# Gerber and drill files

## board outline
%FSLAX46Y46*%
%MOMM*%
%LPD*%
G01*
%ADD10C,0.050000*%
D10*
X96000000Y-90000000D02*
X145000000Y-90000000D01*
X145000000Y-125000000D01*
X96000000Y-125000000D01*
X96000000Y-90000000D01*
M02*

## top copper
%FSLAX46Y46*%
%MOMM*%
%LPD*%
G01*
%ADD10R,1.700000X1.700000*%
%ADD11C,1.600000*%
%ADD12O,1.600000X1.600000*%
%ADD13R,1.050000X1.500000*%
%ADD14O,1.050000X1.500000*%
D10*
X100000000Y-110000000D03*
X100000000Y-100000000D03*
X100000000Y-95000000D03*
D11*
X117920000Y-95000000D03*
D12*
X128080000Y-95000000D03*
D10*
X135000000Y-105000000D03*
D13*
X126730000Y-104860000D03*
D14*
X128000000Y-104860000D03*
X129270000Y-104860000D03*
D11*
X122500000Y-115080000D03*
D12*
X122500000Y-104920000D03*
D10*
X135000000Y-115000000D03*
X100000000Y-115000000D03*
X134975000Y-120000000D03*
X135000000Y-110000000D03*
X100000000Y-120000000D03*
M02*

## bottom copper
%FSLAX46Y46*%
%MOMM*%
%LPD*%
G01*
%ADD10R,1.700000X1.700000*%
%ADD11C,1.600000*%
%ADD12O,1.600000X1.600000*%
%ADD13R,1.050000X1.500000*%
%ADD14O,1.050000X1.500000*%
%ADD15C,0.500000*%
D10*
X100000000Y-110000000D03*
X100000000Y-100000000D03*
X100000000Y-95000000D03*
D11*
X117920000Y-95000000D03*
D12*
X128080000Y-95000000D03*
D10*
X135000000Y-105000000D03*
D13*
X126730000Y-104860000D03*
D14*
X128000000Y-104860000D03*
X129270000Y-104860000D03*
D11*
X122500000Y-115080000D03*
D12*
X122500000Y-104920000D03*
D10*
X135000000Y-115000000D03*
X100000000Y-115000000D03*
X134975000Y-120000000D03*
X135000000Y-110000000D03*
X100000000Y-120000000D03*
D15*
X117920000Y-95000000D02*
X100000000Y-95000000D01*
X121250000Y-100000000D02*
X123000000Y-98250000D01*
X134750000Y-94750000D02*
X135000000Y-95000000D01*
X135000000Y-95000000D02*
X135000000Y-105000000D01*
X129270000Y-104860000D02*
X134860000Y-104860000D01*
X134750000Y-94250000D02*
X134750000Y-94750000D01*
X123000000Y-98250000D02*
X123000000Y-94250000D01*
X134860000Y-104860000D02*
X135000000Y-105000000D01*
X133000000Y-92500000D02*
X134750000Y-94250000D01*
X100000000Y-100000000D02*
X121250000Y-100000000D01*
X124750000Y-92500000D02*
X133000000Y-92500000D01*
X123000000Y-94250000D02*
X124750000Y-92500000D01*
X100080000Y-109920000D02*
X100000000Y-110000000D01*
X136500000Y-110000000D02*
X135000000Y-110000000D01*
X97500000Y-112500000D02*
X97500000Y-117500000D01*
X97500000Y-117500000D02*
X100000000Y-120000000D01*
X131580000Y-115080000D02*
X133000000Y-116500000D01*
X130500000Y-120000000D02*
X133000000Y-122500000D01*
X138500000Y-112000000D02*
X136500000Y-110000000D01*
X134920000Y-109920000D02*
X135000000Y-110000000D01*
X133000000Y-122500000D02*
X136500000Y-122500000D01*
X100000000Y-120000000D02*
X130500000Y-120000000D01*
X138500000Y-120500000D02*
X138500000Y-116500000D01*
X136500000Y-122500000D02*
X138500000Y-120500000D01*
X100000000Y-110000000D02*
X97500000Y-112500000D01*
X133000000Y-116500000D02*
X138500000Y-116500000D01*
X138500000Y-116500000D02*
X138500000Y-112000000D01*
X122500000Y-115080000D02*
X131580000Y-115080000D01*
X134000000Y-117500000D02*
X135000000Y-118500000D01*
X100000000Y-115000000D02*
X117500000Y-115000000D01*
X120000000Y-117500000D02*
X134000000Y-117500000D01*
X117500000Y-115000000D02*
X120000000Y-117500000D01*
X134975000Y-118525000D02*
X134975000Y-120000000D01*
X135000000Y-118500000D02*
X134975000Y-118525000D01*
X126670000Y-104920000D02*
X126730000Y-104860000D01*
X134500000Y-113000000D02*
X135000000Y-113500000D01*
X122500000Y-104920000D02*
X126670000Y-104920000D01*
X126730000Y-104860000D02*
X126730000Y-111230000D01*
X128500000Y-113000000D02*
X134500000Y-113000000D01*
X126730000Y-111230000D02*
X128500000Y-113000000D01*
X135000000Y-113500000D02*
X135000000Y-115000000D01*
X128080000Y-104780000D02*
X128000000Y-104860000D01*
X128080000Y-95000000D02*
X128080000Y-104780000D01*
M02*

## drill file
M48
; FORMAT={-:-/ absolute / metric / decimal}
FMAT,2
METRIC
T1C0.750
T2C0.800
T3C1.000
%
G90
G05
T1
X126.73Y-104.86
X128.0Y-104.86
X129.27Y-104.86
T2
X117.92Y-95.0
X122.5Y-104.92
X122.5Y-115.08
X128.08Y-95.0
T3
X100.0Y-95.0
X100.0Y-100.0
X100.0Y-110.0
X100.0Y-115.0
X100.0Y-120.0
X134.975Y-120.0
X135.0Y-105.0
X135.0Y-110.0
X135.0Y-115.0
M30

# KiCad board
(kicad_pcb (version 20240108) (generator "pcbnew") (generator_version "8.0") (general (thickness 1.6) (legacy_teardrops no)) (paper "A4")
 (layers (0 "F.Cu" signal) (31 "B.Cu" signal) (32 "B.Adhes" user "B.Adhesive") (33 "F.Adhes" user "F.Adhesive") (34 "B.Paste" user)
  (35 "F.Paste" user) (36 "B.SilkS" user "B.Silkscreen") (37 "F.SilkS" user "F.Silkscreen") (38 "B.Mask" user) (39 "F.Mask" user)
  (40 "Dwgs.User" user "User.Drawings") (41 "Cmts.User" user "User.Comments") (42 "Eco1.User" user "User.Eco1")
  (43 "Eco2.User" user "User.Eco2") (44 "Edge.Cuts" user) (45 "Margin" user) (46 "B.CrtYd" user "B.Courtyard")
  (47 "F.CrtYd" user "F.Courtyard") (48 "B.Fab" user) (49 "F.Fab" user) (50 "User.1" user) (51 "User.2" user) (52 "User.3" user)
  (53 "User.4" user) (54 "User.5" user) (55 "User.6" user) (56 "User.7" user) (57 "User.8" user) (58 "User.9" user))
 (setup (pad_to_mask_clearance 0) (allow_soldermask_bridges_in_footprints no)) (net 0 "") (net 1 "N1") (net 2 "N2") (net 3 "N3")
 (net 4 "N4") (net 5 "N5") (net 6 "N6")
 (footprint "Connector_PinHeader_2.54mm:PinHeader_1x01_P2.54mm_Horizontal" (layer "F.Cu") (at 100 110 180)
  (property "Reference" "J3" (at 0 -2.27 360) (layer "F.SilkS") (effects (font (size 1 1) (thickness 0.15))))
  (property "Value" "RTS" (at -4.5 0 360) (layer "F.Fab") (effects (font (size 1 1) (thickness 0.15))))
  (pad "1" thru_hole rect (at 0 0 180) (size 1.7 1.7) (drill 1) (layers "*.Cu" "*.Mask") (remove_unused_layers no) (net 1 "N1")))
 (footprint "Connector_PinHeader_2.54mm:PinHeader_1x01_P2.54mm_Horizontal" (layer "F.Cu") (at 100 100 180)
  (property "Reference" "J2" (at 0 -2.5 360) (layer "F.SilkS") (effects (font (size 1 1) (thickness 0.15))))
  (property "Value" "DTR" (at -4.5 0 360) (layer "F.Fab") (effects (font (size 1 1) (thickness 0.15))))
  (pad "1" thru_hole rect (at 0 0 180) (size 1.7 1.7) (drill 1) (layers "*.Cu" "*.Mask") (remove_unused_layers no) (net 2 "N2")))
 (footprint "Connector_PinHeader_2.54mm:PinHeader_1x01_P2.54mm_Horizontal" (layer "F.Cu") (at 100 95 180)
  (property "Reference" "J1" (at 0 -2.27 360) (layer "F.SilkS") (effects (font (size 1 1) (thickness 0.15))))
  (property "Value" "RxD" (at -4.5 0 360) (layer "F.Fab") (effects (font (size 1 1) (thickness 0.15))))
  (pad "1" thru_hole rect (at 0 0 180) (size 1.7 1.7) (drill 1) (layers "*.Cu" "*.Mask") (remove_unused_layers no) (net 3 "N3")))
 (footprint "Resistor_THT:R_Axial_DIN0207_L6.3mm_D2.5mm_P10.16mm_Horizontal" (layer "F.Cu") (at 117.92 95)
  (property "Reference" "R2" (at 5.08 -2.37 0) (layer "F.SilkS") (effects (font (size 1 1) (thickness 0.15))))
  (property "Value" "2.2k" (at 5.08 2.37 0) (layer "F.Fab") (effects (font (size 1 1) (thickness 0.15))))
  (pad "1" thru_hole circle (at 0 0) (size 1.6 1.6) (drill 0.8) (layers "*.Cu" "*.Mask") (remove_unused_layers no) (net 3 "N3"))
  (pad "2" thru_hole oval (at 10.16 0) (size 1.6 1.6) (drill 0.8) (layers "*.Cu" "*.Mask") (remove_unused_layers no) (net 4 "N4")))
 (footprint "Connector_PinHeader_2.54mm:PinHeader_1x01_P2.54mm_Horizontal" (layer "F.Cu") (at 135 105)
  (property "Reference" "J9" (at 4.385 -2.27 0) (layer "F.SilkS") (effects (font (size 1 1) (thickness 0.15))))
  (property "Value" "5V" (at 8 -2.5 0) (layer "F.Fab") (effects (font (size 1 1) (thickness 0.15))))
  (pad "1" thru_hole rect (at 0 0) (size 1.7 1.7) (drill 1) (layers "*.Cu" "*.Mask") (remove_unused_layers no) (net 2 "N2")))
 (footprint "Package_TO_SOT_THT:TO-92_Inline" (layer "F.Cu") (at 126.73 104.86)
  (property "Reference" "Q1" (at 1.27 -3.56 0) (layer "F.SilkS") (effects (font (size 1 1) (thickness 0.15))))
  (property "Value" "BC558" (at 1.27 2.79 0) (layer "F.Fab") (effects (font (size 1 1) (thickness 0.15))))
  (pad "1" thru_hole rect (at 0 0) (size 1.05 1.5) (drill 0.75) (layers "*.Cu" "*.Mask") (remove_unused_layers no) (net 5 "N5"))
  (pad "2" thru_hole oval (at 1.27 0) (size 1.05 1.5) (drill 0.75) (layers "*.Cu" "*.Mask") (remove_unused_layers no) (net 4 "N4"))
  (pad "3" thru_hole oval (at 2.54 0) (size 1.05 1.5) (drill 0.75) (layers "*.Cu" "*.Mask") (remove_unused_layers no) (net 2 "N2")))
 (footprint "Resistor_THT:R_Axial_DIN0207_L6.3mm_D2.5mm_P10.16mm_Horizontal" (layer "F.Cu") (at 122.5 115.08 90)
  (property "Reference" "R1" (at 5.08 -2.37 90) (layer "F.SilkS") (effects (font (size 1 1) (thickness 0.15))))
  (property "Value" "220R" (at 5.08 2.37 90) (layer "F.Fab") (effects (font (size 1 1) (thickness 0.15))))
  (pad "1" thru_hole circle (at 0 0 90) (size 1.6 1.6) (drill 0.8) (layers "*.Cu" "*.Mask") (remove_unused_layers no) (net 1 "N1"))
  (pad "2" thru_hole oval (at 10.16 0 90) (size 1.6 1.6) (drill 0.8) (layers "*.Cu" "*.Mask") (remove_unused_layers no) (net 5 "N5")))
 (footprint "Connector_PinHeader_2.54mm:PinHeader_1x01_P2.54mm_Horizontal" (layer "F.Cu") (at 135 115)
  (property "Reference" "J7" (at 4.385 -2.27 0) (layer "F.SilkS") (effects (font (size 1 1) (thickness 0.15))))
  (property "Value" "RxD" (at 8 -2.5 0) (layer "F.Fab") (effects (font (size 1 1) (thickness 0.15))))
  (pad "1" thru_hole rect (at 0 0) (size 1.7 1.7) (drill 1) (layers "*.Cu" "*.Mask") (remove_unused_layers no) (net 5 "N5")))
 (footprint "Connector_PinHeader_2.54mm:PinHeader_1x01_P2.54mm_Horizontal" (layer "F.Cu") (at 100 115 180)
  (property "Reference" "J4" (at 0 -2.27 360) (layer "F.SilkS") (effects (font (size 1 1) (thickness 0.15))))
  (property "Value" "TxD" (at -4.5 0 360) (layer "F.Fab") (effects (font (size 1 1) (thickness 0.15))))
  (pad "1" thru_hole rect (at 0 0 180) (size 1.7 1.7) (drill 1) (layers "*.Cu" "*.Mask") (remove_unused_layers no) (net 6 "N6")))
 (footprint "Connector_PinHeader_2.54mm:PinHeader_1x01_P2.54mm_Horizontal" (layer "F.Cu") (at 134.975 120)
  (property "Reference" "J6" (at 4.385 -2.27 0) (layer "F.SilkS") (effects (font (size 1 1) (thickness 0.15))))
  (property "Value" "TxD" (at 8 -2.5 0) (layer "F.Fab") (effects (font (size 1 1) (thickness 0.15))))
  (pad "1" thru_hole rect (at 0 0) (size 1.7 1.7) (drill 1) (layers "*.Cu" "*.Mask") (remove_unused_layers no) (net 6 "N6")))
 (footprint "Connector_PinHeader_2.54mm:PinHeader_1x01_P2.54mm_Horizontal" (layer "F.Cu") (at 135 110)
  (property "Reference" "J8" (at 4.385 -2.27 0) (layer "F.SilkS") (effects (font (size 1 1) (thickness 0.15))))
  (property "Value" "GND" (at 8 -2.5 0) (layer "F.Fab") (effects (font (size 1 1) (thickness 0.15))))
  (pad "1" thru_hole rect (at 0 0) (size 1.7 1.7) (drill 1) (layers "*.Cu" "*.Mask") (remove_unused_layers no) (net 1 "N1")))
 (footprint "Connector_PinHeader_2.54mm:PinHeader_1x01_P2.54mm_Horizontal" (layer "F.Cu") (at 100 120 180)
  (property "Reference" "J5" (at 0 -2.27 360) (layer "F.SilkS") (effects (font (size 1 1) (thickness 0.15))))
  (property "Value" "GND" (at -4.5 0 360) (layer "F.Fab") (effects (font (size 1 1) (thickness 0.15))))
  (pad "1" thru_hole rect (at 0 0 180) (size 1.7 1.7) (drill 1) (layers "*.Cu" "*.Mask") (remove_unused_layers no) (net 1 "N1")))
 (gr_rect (start 96 90) (end 145 125) (stroke (width 0.05) (type default)) (fill none) (layer "Edge.Cuts"))
 (segment (start 117.92 95) (end 100 95) (width 0.5) (layer "B.Cu") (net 3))
 (segment (start 121.25 100) (end 123 98.25) (width 0.5) (layer "B.Cu") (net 2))
 (segment (start 134.75 94.75) (end 135 95) (width 0.5) (layer "B.Cu") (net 2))
 (segment (start 135 95) (end 135 105) (width 0.5) (layer "B.Cu") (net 2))
 (segment (start 129.27 104.86) (end 134.86 104.86) (width 0.5) (layer "B.Cu") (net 2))
 (segment (start 134.75 94.25) (end 134.75 94.75) (width 0.5) (layer "B.Cu") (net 2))
 (segment (start 123 98.25) (end 123 94.25) (width 0.5) (layer "B.Cu") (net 2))
 (segment (start 134.86 104.86) (end 135 105) (width 0.5) (layer "B.Cu") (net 2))
 (segment (start 133 92.5) (end 134.75 94.25) (width 0.5) (layer "B.Cu") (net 2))
 (segment (start 100 100) (end 121.25 100) (width 0.5) (layer "B.Cu") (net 2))
 (segment (start 124.75 92.5) (end 133 92.5) (width 0.5) (layer "B.Cu") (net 2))
 (segment (start 123 94.25) (end 124.75 92.5) (width 0.5) (layer "B.Cu") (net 2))
 (segment (start 100.08 109.92) (end 100 110) (width 0.5) (layer "B.Cu") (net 1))
 (segment (start 136.5 110) (end 135 110) (width 0.5) (layer "B.Cu") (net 1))
 (segment (start 97.5 112.5) (end 97.5 117.5) (width 0.5) (layer "B.Cu") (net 1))
 (segment (start 97.5 117.5) (end 100 120) (width 0.5) (layer "B.Cu") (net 1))
 (segment (start 131.58 115.08) (end 133 116.5) (width 0.5) (layer "B.Cu") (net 1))
 (segment (start 130.5 120) (end 133 122.5) (width 0.5) (layer "B.Cu") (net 1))
 (segment (start 138.5 112) (end 136.5 110) (width 0.5) (layer "B.Cu") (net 1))
 (segment (start 134.92 109.92) (end 135 110) (width 0.5) (layer "B.Cu") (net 1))
 (segment (start 133 122.5) (end 136.5 122.5) (width 0.5) (layer "B.Cu") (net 1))
 (segment (start 100 120) (end 130.5 120) (width 0.5) (layer "B.Cu") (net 1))
 (segment (start 138.5 120.5) (end 138.5 116.5) (width 0.5) (layer "B.Cu") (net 1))
 (segment (start 136.5 122.5) (end 138.5 120.5) (width 0.5) (layer "B.Cu") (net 1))
 (segment (start 100 110) (end 97.5 112.5) (width 0.5) (layer "B.Cu") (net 1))
 (segment (start 133 116.5) (end 138.5 116.5) (width 0.5) (layer "B.Cu") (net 1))
 (segment (start 138.5 116.5) (end 138.5 112) (width 0.5) (layer "B.Cu") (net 1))
 (segment (start 122.5 115.08) (end 131.58 115.08) (width 0.5) (layer "B.Cu") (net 1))
 (segment (start 134 117.5) (end 135 118.5) (width 0.5) (layer "B.Cu") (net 6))
 (segment (start 100 115) (end 117.5 115) (width 0.5) (layer "B.Cu") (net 6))
 (segment (start 120 117.5) (end 134 117.5) (width 0.5) (layer "B.Cu") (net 6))
 (segment (start 117.5 115) (end 120 117.5) (width 0.5) (layer "B.Cu") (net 6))
 (segment (start 134.975 118.525) (end 134.975 120) (width 0.5) (layer "B.Cu") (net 6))
 (segment (start 135 118.5) (end 134.975 118.525) (width 0.5) (layer "B.Cu") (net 6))
 (segment (start 126.67 104.92) (end 126.73 104.86) (width 0.5) (layer "B.Cu") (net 5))
 (segment (start 134.5 113) (end 135 113.5) (width 0.5) (layer "B.Cu") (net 5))
 (segment (start 122.5 104.92) (end 126.67 104.92) (width 0.5) (layer "B.Cu") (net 5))
 (segment (start 126.73 104.86) (end 126.73 111.23) (width 0.5) (layer "B.Cu") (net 5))
 (segment (start 128.5 113) (end 134.5 113) (width 0.5) (layer "B.Cu") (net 5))
 (segment (start 126.73 111.23) (end 128.5 113) (width 0.5) (layer "B.Cu") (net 5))
 (segment (start 135 113.5) (end 135 115) (width 0.5) (layer "B.Cu") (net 5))
 (segment (start 128.08 104.78) (end 128 104.86) (width 0.5) (layer "B.Cu") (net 4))
 (segment (start 128.08 95) (end 128.08 104.78) (width 0.5) (layer "B.Cu") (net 4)))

